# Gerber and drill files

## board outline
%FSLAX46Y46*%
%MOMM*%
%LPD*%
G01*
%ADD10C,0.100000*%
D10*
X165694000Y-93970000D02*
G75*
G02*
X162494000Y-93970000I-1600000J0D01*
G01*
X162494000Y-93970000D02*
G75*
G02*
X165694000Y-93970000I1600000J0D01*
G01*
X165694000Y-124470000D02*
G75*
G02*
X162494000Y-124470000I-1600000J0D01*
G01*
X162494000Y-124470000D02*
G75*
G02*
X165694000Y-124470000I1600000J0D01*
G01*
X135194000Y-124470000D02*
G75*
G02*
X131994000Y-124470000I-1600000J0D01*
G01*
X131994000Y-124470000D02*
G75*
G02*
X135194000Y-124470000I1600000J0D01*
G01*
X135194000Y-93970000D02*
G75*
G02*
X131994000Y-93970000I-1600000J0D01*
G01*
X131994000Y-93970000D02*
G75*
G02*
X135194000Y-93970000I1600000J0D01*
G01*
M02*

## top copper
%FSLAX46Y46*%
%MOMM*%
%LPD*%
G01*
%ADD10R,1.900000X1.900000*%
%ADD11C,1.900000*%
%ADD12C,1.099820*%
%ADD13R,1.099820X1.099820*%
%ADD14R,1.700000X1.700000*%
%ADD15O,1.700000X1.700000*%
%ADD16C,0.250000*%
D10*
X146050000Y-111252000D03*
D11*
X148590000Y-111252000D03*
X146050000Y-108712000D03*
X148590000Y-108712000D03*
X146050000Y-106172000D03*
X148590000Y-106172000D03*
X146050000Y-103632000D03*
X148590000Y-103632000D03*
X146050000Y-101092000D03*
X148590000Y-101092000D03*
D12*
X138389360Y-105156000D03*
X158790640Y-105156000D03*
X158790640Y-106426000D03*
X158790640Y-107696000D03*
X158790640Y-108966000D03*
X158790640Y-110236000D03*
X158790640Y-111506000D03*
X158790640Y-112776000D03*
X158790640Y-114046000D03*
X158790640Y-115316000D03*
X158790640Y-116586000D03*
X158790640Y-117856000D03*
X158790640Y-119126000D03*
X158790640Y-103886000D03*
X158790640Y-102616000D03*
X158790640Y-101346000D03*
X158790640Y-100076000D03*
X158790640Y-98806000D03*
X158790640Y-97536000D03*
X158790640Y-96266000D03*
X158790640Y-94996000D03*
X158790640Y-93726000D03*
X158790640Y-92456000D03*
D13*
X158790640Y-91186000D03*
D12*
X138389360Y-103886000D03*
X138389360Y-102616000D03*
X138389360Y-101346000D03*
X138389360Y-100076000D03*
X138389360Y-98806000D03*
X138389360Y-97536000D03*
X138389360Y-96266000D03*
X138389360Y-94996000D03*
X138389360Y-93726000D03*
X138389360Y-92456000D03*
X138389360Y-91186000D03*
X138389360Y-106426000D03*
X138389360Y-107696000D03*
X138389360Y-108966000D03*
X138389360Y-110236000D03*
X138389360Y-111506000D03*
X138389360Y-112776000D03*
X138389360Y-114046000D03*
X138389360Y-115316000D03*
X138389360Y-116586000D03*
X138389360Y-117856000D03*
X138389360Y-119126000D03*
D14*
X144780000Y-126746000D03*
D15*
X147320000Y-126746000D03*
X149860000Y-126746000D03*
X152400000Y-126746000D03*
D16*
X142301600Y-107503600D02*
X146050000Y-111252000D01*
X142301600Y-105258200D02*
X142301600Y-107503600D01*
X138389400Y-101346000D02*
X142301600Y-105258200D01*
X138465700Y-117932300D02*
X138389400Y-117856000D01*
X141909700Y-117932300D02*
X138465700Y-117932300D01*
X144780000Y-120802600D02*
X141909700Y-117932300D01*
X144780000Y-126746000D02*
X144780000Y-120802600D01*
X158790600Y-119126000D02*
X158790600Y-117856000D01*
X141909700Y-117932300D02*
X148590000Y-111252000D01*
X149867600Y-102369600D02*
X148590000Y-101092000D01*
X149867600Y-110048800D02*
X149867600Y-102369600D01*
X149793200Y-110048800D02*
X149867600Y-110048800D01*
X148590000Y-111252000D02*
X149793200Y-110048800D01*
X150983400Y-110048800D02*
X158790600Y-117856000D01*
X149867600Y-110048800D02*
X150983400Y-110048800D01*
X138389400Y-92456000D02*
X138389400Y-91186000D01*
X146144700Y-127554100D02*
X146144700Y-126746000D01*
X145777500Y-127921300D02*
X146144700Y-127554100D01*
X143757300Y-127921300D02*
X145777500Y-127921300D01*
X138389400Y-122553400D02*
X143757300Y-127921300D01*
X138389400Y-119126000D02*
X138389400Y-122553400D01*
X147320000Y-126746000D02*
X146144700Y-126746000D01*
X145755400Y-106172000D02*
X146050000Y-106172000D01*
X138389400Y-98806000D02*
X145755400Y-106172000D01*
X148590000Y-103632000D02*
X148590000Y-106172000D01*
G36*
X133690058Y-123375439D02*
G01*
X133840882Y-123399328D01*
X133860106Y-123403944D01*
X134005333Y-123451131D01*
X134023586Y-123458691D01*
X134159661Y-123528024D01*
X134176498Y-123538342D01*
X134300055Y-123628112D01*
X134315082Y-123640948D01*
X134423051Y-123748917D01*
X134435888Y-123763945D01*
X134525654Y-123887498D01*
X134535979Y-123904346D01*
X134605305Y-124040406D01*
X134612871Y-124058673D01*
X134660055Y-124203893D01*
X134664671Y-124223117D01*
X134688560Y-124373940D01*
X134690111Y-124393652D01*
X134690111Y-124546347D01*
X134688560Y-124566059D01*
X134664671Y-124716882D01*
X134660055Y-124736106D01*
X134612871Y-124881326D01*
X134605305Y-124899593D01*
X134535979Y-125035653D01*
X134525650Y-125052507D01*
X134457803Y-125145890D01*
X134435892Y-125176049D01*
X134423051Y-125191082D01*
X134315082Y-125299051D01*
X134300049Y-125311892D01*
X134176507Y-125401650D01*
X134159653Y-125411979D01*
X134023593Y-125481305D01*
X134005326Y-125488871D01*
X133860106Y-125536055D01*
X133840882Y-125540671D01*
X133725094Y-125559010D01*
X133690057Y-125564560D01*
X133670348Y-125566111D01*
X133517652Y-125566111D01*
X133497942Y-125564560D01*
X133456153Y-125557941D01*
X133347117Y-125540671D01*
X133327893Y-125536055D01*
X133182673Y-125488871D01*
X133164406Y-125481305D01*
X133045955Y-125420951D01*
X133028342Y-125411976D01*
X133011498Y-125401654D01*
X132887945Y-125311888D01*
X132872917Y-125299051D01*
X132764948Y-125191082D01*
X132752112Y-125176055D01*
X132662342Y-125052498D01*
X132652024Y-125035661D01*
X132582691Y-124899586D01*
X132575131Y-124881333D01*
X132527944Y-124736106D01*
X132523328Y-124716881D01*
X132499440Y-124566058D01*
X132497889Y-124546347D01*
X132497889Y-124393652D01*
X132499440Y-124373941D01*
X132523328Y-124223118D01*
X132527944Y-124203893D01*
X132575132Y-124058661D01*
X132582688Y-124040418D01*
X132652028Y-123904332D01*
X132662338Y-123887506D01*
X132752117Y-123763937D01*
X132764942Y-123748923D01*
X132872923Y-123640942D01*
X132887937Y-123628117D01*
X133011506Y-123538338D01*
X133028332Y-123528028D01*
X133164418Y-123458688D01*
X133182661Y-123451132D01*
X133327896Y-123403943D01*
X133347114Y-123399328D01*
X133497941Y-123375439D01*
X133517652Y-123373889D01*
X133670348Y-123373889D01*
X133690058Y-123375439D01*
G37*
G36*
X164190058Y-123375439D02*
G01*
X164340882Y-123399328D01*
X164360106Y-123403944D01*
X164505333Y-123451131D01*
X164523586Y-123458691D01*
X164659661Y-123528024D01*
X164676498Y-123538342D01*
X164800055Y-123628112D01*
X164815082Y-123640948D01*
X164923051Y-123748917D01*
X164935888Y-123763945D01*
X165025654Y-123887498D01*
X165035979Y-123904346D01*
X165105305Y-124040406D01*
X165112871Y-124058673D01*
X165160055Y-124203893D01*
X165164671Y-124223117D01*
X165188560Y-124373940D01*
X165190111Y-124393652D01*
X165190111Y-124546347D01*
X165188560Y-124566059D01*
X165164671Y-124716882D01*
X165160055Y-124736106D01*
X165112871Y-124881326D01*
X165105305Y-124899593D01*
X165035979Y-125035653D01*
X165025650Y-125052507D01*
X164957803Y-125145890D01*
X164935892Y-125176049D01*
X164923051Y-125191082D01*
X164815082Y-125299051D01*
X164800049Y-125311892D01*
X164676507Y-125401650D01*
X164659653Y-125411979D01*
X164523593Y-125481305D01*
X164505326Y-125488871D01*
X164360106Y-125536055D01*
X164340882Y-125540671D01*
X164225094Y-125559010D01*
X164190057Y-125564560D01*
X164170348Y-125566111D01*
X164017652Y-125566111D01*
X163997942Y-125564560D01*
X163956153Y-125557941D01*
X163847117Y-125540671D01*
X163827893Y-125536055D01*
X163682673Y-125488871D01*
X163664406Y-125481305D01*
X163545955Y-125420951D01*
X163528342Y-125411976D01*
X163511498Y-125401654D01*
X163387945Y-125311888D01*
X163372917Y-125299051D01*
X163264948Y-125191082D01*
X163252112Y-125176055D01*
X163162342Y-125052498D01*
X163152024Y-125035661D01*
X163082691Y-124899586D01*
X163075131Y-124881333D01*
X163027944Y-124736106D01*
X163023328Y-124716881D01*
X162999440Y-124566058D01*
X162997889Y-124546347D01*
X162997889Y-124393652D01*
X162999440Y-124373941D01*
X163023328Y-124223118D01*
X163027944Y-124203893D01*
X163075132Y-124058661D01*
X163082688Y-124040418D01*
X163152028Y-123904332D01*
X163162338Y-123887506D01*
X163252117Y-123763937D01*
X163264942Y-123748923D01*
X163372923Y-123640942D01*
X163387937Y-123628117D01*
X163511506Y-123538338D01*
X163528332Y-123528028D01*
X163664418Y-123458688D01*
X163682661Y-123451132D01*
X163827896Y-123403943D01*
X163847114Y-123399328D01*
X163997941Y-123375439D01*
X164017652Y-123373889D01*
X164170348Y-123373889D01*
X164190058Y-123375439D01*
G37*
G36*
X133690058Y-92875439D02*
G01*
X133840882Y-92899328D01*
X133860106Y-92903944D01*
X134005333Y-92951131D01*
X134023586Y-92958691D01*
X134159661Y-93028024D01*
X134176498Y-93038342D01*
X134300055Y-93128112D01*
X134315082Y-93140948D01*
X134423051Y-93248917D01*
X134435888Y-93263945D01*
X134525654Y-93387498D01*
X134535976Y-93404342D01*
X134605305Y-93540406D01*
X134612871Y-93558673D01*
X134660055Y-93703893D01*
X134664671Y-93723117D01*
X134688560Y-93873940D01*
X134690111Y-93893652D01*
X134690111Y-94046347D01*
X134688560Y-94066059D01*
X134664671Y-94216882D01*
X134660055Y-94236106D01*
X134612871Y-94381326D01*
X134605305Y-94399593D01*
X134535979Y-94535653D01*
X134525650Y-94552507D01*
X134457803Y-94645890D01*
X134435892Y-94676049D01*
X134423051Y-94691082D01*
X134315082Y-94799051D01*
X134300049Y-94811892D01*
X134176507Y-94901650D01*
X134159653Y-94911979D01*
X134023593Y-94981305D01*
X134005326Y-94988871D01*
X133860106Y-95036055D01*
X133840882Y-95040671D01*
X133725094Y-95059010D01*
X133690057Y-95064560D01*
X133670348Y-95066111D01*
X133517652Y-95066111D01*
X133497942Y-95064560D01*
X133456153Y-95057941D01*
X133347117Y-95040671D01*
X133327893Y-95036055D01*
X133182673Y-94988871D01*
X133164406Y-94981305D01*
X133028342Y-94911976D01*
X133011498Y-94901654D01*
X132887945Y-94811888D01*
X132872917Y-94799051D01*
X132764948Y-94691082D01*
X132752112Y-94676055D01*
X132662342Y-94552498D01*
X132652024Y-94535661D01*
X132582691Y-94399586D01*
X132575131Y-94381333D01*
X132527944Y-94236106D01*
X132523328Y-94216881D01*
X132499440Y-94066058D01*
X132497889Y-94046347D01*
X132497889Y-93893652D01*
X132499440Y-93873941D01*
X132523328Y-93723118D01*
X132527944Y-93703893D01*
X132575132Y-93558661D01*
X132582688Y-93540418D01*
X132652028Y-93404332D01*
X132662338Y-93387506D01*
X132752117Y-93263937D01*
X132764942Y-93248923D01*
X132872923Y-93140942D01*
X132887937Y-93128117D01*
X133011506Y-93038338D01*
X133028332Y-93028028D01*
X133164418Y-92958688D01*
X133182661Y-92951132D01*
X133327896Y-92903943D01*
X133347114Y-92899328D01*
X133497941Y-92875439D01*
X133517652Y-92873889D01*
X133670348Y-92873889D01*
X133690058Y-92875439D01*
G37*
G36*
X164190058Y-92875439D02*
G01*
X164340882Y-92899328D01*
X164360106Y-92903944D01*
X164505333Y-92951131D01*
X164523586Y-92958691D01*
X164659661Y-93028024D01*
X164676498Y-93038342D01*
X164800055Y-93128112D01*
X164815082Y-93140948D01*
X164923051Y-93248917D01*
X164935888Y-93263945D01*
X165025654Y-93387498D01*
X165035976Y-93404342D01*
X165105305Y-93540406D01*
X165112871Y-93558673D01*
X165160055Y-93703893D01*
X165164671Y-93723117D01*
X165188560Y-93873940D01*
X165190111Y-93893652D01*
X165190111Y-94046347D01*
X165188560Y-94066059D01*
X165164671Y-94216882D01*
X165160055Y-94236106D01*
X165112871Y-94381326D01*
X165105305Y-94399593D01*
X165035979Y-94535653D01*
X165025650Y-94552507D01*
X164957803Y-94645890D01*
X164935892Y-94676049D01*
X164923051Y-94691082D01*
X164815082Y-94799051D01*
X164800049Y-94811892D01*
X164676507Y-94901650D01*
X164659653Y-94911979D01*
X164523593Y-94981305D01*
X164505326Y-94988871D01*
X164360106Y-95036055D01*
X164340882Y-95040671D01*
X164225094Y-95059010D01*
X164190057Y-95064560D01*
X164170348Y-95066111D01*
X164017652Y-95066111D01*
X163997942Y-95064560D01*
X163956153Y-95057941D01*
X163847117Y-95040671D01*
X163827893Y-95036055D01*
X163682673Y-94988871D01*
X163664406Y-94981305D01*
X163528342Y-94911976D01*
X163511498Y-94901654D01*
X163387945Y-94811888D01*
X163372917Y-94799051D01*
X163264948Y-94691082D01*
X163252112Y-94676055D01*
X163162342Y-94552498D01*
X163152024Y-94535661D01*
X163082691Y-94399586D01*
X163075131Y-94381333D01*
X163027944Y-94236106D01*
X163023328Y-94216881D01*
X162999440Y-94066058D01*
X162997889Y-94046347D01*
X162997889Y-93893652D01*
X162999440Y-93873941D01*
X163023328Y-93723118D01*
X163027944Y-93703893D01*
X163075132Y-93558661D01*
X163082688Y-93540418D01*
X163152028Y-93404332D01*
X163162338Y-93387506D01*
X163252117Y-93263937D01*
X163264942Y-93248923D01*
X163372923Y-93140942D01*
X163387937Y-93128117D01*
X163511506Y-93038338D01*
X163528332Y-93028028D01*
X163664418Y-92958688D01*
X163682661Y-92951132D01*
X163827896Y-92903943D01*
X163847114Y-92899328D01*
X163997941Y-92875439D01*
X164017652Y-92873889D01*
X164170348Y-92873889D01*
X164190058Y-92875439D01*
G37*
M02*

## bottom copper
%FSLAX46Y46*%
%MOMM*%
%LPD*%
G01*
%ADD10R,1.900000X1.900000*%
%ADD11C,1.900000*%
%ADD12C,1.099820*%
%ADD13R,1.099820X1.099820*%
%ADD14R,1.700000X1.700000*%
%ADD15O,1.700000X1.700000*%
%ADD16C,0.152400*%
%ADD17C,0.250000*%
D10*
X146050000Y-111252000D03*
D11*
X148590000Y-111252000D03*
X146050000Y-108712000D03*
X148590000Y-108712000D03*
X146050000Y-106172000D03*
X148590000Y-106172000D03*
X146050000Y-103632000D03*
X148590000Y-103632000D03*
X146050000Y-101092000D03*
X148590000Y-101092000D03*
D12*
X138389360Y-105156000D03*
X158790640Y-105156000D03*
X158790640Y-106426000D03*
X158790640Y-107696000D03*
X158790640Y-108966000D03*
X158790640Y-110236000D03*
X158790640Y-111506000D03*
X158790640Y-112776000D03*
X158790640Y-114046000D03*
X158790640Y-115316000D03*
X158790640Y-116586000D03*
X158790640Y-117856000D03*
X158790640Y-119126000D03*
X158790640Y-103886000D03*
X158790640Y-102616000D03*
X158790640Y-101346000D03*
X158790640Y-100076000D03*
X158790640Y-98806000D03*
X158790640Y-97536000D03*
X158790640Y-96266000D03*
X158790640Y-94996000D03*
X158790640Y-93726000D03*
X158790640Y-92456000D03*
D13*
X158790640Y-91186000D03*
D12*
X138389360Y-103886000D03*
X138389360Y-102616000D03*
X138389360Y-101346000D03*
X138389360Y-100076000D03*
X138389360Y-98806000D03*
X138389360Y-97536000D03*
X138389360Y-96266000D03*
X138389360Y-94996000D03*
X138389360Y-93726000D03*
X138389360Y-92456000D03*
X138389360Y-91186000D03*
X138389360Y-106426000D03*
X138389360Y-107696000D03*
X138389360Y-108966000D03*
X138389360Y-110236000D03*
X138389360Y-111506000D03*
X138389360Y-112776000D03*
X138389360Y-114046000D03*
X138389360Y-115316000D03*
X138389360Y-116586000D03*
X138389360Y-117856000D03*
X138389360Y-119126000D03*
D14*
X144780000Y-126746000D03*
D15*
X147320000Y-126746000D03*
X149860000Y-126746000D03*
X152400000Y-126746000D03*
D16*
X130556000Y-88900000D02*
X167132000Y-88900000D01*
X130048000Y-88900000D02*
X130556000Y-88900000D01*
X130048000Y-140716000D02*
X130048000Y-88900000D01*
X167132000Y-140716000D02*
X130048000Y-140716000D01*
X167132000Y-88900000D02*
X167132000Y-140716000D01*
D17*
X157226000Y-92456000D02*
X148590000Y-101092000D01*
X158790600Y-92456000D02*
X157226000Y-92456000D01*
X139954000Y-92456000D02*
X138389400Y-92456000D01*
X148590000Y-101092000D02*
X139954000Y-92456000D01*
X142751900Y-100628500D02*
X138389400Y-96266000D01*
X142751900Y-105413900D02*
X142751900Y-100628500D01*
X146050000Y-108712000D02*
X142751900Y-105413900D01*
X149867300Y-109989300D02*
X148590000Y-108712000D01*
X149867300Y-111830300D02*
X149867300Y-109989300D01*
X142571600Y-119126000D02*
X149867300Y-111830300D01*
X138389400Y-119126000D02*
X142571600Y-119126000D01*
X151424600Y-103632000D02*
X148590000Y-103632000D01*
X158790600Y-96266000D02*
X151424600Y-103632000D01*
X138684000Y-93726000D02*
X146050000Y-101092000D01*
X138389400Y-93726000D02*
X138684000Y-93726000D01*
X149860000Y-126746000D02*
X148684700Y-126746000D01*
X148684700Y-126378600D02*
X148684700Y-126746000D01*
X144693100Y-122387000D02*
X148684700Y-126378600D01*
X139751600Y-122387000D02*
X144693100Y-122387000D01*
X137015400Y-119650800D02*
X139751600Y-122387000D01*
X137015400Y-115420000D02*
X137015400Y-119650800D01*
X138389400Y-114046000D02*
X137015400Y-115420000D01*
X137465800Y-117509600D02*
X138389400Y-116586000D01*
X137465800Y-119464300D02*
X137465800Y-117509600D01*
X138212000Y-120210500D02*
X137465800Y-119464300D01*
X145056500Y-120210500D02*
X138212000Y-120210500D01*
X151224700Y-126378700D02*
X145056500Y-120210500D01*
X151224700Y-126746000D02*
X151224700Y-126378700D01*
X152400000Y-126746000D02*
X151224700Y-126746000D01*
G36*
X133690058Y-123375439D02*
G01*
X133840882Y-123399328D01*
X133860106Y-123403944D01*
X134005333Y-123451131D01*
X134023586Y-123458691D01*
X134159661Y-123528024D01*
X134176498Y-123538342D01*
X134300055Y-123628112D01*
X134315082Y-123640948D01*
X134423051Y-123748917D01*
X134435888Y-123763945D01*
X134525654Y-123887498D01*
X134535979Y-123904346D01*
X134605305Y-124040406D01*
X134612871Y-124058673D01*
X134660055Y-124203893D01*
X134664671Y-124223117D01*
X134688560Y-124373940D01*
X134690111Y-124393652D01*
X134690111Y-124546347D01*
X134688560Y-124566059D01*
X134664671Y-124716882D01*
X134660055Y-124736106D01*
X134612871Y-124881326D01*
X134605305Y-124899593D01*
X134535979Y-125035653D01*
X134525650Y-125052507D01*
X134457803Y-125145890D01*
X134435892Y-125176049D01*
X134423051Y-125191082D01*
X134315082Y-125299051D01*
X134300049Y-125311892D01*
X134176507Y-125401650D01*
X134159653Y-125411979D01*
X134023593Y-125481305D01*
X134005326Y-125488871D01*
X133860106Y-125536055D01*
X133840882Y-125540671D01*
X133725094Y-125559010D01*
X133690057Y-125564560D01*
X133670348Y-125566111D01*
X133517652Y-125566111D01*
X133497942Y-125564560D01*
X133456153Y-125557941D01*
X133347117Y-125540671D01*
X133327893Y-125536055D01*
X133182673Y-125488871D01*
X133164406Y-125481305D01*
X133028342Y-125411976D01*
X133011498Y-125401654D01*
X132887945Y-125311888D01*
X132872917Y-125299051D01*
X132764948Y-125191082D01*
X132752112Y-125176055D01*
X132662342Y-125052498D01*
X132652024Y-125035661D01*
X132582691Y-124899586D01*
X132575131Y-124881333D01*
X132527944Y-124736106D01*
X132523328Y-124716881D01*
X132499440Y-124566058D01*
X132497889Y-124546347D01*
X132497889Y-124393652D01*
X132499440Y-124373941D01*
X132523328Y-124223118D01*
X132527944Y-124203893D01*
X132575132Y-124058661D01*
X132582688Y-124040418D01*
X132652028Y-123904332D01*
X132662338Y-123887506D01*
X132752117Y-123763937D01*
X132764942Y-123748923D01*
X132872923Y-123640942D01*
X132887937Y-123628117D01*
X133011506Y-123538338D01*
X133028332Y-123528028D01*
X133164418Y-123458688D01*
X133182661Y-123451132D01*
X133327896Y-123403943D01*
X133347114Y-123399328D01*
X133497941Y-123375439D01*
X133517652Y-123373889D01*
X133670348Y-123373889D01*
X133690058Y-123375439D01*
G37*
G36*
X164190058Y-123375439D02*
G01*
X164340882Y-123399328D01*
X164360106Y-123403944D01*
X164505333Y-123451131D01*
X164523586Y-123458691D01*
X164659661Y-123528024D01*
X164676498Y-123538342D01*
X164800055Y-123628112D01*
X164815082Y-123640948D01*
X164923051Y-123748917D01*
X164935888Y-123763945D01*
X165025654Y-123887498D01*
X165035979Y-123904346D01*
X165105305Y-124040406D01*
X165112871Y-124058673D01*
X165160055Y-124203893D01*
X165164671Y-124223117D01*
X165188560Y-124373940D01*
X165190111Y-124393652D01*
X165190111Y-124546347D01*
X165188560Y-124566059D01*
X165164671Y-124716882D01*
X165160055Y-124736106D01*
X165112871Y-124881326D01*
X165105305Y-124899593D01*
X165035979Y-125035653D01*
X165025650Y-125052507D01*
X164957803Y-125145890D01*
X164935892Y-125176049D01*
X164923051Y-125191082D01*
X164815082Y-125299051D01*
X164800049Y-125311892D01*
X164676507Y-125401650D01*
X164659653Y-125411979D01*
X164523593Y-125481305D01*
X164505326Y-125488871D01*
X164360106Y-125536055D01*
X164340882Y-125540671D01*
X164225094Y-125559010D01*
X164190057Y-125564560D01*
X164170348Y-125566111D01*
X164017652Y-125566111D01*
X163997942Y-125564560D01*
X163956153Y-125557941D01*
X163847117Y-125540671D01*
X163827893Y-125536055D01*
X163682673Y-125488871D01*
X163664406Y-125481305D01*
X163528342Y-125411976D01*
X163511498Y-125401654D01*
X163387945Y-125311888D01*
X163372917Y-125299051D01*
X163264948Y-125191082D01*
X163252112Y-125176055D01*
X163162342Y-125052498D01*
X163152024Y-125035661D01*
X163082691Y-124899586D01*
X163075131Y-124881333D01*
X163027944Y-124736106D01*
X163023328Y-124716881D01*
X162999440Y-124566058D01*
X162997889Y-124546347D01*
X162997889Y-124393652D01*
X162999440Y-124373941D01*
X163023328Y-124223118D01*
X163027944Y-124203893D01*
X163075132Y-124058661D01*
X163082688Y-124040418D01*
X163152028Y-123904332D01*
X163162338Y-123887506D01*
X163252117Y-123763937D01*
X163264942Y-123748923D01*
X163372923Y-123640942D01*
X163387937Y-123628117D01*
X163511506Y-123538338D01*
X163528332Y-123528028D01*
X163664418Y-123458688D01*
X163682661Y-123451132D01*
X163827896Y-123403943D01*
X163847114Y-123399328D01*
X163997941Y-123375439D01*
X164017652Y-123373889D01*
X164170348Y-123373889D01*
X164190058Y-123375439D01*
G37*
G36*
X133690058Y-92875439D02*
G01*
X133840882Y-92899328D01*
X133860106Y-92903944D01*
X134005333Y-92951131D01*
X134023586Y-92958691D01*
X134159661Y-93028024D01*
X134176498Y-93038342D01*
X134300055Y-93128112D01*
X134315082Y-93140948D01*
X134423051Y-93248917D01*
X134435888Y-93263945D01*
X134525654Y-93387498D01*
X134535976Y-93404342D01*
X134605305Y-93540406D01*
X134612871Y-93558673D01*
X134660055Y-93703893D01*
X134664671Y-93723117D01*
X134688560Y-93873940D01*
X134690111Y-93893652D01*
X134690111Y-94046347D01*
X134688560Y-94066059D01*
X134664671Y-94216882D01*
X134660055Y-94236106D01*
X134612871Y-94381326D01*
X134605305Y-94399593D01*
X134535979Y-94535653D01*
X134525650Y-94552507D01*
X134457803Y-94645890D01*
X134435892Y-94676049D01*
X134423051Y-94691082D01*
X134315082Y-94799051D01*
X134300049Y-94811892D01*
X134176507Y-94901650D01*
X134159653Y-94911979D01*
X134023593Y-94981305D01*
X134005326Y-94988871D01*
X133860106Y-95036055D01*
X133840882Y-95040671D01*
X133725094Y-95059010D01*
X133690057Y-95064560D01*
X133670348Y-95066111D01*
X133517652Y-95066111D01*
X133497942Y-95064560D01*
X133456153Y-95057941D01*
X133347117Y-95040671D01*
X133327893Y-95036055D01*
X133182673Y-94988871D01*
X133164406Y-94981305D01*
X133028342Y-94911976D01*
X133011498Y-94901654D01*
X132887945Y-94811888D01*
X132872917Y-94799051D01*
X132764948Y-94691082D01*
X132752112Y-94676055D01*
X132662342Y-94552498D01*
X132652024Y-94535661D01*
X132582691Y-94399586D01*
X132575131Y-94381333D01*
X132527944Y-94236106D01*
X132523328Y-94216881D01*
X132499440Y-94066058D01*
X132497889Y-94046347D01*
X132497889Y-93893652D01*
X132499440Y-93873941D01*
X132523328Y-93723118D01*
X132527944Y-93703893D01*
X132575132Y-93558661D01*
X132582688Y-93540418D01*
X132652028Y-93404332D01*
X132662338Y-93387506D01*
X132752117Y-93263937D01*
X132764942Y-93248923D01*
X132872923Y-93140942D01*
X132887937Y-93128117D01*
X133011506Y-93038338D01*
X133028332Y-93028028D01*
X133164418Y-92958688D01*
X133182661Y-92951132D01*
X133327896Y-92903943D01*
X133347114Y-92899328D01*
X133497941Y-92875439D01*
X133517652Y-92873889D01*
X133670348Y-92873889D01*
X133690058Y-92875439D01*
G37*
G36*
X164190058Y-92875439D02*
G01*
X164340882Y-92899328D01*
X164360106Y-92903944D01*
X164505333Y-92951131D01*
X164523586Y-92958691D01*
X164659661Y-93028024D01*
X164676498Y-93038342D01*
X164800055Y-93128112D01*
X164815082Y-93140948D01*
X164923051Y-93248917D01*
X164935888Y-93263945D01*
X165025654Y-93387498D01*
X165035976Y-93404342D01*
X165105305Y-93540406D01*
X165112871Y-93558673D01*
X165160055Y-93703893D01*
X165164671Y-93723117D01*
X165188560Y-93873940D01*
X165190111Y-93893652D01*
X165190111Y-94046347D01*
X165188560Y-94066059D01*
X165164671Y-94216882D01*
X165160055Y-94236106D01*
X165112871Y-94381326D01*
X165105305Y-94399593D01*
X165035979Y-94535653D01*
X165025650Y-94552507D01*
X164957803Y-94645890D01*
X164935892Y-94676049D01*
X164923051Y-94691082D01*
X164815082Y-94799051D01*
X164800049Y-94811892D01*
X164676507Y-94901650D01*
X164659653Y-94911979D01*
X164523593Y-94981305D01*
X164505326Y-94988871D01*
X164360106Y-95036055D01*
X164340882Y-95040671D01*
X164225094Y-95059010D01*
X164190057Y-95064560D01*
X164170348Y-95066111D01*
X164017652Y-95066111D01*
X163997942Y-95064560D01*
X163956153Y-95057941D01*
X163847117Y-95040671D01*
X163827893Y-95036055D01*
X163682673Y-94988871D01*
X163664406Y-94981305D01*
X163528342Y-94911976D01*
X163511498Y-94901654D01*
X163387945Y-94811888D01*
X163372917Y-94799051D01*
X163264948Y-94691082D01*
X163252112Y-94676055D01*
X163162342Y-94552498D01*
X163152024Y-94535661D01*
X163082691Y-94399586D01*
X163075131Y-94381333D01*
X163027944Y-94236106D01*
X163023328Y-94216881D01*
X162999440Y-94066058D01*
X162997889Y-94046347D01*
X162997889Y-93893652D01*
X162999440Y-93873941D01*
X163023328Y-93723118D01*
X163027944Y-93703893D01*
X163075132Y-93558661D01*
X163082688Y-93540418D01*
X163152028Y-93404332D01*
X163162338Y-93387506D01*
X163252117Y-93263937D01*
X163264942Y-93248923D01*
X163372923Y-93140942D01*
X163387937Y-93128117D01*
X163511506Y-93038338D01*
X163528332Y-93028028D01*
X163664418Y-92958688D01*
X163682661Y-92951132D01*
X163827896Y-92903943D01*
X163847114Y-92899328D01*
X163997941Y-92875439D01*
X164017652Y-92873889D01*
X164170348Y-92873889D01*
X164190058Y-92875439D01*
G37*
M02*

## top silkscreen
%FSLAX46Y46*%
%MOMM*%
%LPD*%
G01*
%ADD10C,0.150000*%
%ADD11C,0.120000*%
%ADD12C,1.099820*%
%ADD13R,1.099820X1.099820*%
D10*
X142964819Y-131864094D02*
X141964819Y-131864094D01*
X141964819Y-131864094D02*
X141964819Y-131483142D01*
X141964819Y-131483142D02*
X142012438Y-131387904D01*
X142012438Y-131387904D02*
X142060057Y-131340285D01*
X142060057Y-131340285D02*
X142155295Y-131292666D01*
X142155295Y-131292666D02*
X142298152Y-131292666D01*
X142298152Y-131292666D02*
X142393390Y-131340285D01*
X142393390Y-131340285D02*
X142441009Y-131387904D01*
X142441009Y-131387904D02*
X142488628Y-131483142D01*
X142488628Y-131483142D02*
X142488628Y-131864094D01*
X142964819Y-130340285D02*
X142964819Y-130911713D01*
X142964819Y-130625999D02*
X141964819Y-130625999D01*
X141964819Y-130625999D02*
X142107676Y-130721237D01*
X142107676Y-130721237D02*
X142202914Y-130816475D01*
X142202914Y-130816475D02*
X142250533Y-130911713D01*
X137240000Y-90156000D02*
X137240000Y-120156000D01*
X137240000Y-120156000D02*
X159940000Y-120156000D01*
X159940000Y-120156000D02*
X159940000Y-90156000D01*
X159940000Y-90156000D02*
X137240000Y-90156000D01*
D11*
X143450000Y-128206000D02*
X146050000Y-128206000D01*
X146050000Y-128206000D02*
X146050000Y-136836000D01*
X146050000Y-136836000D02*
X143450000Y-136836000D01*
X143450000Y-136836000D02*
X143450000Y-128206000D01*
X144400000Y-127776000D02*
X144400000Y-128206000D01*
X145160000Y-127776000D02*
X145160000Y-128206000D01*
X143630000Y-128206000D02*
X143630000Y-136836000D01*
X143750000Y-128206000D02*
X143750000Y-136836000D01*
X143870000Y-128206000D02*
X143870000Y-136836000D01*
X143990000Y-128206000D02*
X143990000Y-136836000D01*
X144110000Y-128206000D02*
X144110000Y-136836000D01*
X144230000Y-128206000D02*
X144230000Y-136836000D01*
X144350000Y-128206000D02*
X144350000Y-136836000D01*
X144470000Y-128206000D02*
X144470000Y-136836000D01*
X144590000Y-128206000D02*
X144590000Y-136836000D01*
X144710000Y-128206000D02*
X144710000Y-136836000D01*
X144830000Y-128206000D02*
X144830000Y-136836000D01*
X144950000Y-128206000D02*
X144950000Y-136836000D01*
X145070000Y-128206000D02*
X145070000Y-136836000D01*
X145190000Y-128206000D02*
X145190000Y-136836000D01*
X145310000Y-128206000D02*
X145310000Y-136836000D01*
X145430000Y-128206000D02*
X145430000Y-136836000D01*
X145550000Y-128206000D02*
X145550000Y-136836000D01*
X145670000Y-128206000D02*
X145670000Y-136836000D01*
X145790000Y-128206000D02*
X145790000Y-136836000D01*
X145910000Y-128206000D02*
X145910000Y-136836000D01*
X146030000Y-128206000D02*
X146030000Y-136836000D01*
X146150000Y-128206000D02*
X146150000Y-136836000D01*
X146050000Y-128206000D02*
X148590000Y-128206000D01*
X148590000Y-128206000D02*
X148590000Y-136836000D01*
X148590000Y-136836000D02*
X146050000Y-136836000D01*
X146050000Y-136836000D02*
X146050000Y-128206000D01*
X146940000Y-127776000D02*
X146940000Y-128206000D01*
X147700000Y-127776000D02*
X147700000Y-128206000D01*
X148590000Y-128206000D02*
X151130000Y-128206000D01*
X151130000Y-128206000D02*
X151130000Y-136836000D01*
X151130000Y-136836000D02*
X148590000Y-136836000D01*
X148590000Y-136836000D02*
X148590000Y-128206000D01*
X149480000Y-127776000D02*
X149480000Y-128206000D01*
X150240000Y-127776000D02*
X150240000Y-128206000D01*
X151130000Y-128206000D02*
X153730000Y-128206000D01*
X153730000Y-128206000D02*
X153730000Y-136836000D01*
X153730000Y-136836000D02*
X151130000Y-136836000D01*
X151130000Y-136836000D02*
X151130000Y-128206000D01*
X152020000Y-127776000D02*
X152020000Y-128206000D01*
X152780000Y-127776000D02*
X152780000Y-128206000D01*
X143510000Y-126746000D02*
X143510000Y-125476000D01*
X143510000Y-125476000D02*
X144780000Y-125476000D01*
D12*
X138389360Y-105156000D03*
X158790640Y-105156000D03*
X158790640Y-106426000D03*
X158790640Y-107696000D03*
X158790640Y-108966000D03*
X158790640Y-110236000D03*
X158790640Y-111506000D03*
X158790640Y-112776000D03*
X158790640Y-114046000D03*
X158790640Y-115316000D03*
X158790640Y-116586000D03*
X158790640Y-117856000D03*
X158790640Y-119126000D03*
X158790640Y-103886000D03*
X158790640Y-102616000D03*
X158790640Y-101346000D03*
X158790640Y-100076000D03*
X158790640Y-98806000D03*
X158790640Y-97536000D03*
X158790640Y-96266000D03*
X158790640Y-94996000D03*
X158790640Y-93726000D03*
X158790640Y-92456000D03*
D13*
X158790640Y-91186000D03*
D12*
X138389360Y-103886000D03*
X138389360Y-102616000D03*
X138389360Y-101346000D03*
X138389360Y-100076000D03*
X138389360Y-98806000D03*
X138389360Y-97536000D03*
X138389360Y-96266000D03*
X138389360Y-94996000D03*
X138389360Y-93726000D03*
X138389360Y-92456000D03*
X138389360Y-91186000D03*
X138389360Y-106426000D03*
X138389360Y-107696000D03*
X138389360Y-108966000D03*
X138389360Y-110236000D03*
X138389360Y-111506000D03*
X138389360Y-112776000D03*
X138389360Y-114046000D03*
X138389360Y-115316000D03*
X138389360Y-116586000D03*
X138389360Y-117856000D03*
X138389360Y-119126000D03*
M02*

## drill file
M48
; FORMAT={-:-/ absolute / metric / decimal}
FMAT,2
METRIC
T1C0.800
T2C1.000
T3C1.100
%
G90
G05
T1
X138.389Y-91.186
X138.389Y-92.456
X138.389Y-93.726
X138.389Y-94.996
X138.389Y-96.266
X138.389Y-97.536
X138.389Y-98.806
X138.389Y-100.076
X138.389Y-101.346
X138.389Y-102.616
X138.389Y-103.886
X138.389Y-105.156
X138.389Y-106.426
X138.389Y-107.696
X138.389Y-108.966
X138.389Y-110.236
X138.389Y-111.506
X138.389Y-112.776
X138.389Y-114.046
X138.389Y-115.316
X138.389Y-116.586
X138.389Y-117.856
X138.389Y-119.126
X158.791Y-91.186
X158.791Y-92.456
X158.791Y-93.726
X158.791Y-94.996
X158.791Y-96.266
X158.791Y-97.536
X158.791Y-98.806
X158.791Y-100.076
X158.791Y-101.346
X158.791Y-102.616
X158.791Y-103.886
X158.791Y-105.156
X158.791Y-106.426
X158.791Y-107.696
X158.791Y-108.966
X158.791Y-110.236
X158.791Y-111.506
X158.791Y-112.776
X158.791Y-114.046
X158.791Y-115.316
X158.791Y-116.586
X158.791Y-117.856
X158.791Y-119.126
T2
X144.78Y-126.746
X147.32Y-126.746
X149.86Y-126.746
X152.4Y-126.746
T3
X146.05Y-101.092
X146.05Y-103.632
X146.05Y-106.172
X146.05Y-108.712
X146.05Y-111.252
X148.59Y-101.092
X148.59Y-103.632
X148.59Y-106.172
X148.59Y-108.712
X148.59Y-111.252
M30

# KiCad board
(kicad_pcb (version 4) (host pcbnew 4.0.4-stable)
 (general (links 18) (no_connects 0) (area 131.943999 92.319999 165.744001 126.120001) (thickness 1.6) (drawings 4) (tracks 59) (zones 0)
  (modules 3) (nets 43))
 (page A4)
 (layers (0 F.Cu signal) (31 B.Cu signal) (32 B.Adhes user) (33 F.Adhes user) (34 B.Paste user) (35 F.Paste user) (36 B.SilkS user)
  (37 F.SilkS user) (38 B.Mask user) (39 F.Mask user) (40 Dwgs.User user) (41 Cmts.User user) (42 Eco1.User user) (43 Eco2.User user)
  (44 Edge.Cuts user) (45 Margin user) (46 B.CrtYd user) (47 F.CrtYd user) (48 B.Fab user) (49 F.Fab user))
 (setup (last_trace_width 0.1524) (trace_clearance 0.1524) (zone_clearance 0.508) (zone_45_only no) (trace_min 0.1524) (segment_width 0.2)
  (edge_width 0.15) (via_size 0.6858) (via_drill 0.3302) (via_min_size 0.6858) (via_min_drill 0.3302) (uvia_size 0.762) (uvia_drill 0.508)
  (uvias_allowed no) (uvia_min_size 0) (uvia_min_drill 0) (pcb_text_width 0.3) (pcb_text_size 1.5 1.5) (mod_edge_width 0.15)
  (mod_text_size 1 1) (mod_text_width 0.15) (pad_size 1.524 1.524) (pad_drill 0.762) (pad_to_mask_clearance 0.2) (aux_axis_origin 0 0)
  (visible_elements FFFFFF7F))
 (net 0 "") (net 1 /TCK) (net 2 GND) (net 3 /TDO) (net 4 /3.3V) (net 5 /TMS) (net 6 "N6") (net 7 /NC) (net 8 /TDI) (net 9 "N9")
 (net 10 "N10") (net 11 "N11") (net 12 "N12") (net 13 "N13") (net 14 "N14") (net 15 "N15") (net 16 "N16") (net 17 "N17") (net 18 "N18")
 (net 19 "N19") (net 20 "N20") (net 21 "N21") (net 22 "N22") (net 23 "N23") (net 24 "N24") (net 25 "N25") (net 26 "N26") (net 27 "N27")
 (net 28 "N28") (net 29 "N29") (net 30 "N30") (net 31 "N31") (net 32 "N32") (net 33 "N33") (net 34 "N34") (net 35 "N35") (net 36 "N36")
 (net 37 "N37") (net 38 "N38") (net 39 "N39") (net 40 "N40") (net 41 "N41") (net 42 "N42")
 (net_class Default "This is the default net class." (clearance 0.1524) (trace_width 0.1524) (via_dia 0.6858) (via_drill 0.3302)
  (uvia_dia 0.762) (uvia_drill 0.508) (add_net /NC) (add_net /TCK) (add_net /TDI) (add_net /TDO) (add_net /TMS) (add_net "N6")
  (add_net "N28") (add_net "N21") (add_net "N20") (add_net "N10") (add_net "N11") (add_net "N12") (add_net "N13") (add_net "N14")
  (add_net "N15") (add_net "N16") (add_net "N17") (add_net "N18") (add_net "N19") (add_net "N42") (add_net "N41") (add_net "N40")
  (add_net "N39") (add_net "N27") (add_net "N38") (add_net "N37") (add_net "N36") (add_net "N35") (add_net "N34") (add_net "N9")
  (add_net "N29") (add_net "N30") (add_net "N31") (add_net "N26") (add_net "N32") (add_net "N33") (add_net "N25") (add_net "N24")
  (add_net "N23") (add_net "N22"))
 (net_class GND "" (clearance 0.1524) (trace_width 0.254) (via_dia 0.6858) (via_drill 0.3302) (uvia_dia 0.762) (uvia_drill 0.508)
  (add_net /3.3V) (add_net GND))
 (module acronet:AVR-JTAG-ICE (layer B.Cu) (at 147.32 106.172 90)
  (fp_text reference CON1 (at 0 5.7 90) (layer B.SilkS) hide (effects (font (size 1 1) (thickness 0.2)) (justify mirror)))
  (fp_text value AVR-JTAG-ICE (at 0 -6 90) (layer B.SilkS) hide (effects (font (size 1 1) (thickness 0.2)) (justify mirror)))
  (pad 1 thru_hole rect (at -5.08 -1.27 90) (size 1.9 1.9) (drill 1.1) (layers *.Cu *.Mask B.SilkS) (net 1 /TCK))
  (pad 2 thru_hole circle (at -5.08 1.27 90) (size 1.9 1.9) (drill 1.1) (layers *.Cu *.Mask B.SilkS) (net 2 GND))
  (pad 3 thru_hole circle (at -2.54 -1.27 90) (size 1.9 1.9) (drill 1.1) (layers *.Cu *.Mask B.SilkS) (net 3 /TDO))
  (pad 4 thru_hole circle (at -2.54 1.27 90) (size 1.9 1.9) (drill 1.1) (layers *.Cu *.Mask B.SilkS) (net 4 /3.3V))
  (pad 5 thru_hole circle (at 0 -1.27 90) (size 1.9 1.9) (drill 1.1) (layers *.Cu *.Mask B.SilkS) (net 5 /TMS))
  (pad 6 thru_hole circle (at 0 1.27 90) (size 1.9 1.9) (drill 1.1) (layers *.Cu *.Mask B.SilkS) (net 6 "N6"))
  (pad 7 thru_hole circle (at 2.54 -1.27 90) (size 1.9 1.9) (drill 1.1) (layers *.Cu *.Mask B.SilkS) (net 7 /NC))
  (pad 8 thru_hole circle (at 2.54 1.27 90) (size 1.9 1.9) (drill 1.1) (layers *.Cu *.Mask B.SilkS) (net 6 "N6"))
  (pad 9 thru_hole circle (at 5.08 -1.27 90) (size 1.9 1.9) (drill 1.1) (layers *.Cu *.Mask B.SilkS) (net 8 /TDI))
  (pad 10 thru_hole circle (at 5.08 1.27 90) (size 1.9 1.9) (drill 1.1) (layers *.Cu *.Mask B.SilkS) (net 2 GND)))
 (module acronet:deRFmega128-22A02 (layer F.Cu) (at 148.59 105.156 90)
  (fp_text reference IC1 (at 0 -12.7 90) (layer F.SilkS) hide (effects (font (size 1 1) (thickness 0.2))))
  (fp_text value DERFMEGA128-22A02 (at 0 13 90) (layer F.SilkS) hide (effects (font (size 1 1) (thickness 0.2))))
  (fp_line (start 15 -11.35) (end -15 -11.35) (layer F.SilkS) (width 0.15))
  (fp_line (start -15 -11.35) (end -15 11.35) (layer F.SilkS) (width 0.15))
  (fp_line (start -15 11.35) (end 15 11.35) (layer F.SilkS) (width 0.15))
  (fp_line (start 15 11.35) (end 15 -11.35) (layer F.SilkS) (width 0.15))
  (pad 35 thru_hole circle (at 0 -10.20064 90) (size 1.09982 1.09982) (drill 0.8001) (layers *.Cu *.Mask F.SilkS) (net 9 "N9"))
  (pad 12 thru_hole circle (at 0 10.20064 90) (size 1.09982 1.09982) (drill 0.8001) (layers *.Cu *.Mask F.SilkS) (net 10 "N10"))
  (pad 13 thru_hole circle (at -1.27 10.20064 90) (size 1.09982 1.09982) (drill 0.8001) (layers *.Cu *.Mask F.SilkS) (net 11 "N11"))
  (pad 14 thru_hole circle (at -2.54 10.20064 90) (size 1.09982 1.09982) (drill 0.8001) (layers *.Cu *.Mask F.SilkS) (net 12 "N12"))
  (pad 15 thru_hole circle (at -3.81 10.20064 90) (size 1.09982 1.09982) (drill 0.8001) (layers *.Cu *.Mask F.SilkS) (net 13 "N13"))
  (pad 16 thru_hole circle (at -5.08 10.20064 90) (size 1.09982 1.09982) (drill 0.8001) (layers *.Cu *.Mask F.SilkS) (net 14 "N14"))
  (pad 17 thru_hole circle (at -6.35 10.20064 90) (size 1.09982 1.09982) (drill 0.8001) (layers *.Cu *.Mask F.SilkS) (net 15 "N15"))
  (pad 18 thru_hole circle (at -7.62 10.20064 90) (size 1.09982 1.09982) (drill 0.8001) (layers *.Cu *.Mask F.SilkS) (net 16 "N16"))
  (pad 19 thru_hole circle (at -8.89 10.20064 90) (size 1.09982 1.09982) (drill 0.8001) (layers *.Cu *.Mask F.SilkS) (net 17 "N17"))
  (pad 20 thru_hole circle (at -10.16 10.20064 90) (size 1.09982 1.09982) (drill 0.8001) (layers *.Cu *.Mask F.SilkS) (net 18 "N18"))
  (pad 21 thru_hole circle (at -11.43 10.20064 90) (size 1.09982 1.09982) (drill 0.8001) (layers *.Cu *.Mask F.SilkS) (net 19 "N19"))
  (pad 22 thru_hole circle (at -12.7 10.20064 90) (size 1.09982 1.09982) (drill 0.8001) (layers *.Cu *.Mask F.SilkS) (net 2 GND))
  (pad 23 thru_hole circle (at -13.97 10.20064 90) (size 1.09982 1.09982) (drill 0.8001) (layers *.Cu *.Mask F.SilkS) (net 2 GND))
  (pad 11 thru_hole circle (at 1.27 10.20064 90) (size 1.09982 1.09982) (drill 0.8001) (layers *.Cu *.Mask F.SilkS) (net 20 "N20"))
  (pad 10 thru_hole circle (at 2.54 10.20064 90) (size 1.09982 1.09982) (drill 0.8001) (layers *.Cu *.Mask F.SilkS) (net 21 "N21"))
  (pad 9 thru_hole circle (at 3.81 10.20064 90) (size 1.09982 1.09982) (drill 0.8001) (layers *.Cu *.Mask F.SilkS) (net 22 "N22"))
  (pad 8 thru_hole circle (at 5.08 10.20064 90) (size 1.09982 1.09982) (drill 0.8001) (layers *.Cu *.Mask F.SilkS) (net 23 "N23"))
  (pad 7 thru_hole circle (at 6.35 10.20064 90) (size 1.09982 1.09982) (drill 0.8001) (layers *.Cu *.Mask F.SilkS) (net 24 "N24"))
  (pad 6 thru_hole circle (at 7.62 10.20064 90) (size 1.09982 1.09982) (drill 0.8001) (layers *.Cu *.Mask F.SilkS) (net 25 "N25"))
  (pad 5 thru_hole circle (at 8.89 10.20064 90) (size 1.09982 1.09982) (drill 0.8001) (layers *.Cu *.Mask F.SilkS) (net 6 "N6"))
  (pad 4 thru_hole circle (at 10.16 10.20064 90) (size 1.09982 1.09982) (drill 0.8001) (layers *.Cu *.Mask F.SilkS) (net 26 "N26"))
  (pad 3 thru_hole circle (at 11.43 10.20064 90) (size 1.09982 1.09982) (drill 0.8001) (layers *.Cu *.Mask F.SilkS) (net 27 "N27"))
  (pad 2 thru_hole circle (at 12.7 10.20064 90) (size 1.09982 1.09982) (drill 0.8001) (layers *.Cu *.Mask F.SilkS) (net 2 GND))
  (pad 1 thru_hole rect (at 13.97 10.20064 90) (size 1.09982 1.09982) (drill 0.8001) (layers *.Cu *.Mask F.SilkS) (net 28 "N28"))
  (pad 36 thru_hole circle (at 1.27 -10.20064 90) (size 1.09982 1.09982) (drill 0.8001) (layers *.Cu *.Mask F.SilkS) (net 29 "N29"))
  (pad 37 thru_hole circle (at 2.54 -10.20064 90) (size 1.09982 1.09982) (drill 0.8001) (layers *.Cu *.Mask F.SilkS) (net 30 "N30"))
  (pad 38 thru_hole circle (at 3.81 -10.20064 90) (size 1.09982 1.09982) (drill 0.8001) (layers *.Cu *.Mask F.SilkS) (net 1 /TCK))
  (pad 39 thru_hole circle (at 5.08 -10.20064 90) (size 1.09982 1.09982) (drill 0.8001) (layers *.Cu *.Mask F.SilkS) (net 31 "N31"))
  (pad 40 thru_hole circle (at 6.35 -10.20064 90) (size 1.09982 1.09982) (drill 0.8001) (layers *.Cu *.Mask F.SilkS) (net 5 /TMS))
  (pad 41 thru_hole circle (at 7.62 -10.20064 90) (size 1.09982 1.09982) (drill 0.8001) (layers *.Cu *.Mask F.SilkS) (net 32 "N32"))
  (pad 42 thru_hole circle (at 8.89 -10.20064 90) (size 1.09982 1.09982) (drill 0.8001) (layers *.Cu *.Mask F.SilkS) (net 3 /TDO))
  (pad 43 thru_hole circle (at 10.16 -10.20064 90) (size 1.09982 1.09982) (drill 0.8001) (layers *.Cu *.Mask F.SilkS) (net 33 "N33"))
  (pad 44 thru_hole circle (at 11.43 -10.20064 90) (size 1.09982 1.09982) (drill 0.8001) (layers *.Cu *.Mask F.SilkS) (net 8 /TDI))
  (pad 45 thru_hole circle (at 12.7 -10.20064 90) (size 1.09982 1.09982) (drill 0.8001) (layers *.Cu *.Mask F.SilkS) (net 2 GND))
  (pad 46 thru_hole circle (at 13.97 -10.20064 90) (size 1.09982 1.09982) (drill 0.8001) (layers *.Cu *.Mask F.SilkS) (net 2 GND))
  (pad 34 thru_hole circle (at -1.27 -10.20064 90) (size 1.09982 1.09982) (drill 0.8001) (layers *.Cu *.Mask F.SilkS) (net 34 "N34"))
  (pad 33 thru_hole circle (at -2.54 -10.20064 90) (size 1.09982 1.09982) (drill 0.8001) (layers *.Cu *.Mask F.SilkS) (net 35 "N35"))
  (pad 32 thru_hole circle (at -3.81 -10.20064 90) (size 1.09982 1.09982) (drill 0.8001) (layers *.Cu *.Mask F.SilkS) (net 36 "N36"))
  (pad 31 thru_hole circle (at -5.08 -10.20064 90) (size 1.09982 1.09982) (drill 0.8001) (layers *.Cu *.Mask F.SilkS) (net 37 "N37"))
  (pad 30 thru_hole circle (at -6.35 -10.20064 90) (size 1.09982 1.09982) (drill 0.8001) (layers *.Cu *.Mask F.SilkS) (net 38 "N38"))
  (pad 29 thru_hole circle (at -7.62 -10.20064 90) (size 1.09982 1.09982) (drill 0.8001) (layers *.Cu *.Mask F.SilkS) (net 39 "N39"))
  (pad 28 thru_hole circle (at -8.89 -10.20064 90) (size 1.09982 1.09982) (drill 0.8001) (layers *.Cu *.Mask F.SilkS) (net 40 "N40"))
  (pad 27 thru_hole circle (at -10.16 -10.20064 90) (size 1.09982 1.09982) (drill 0.8001) (layers *.Cu *.Mask F.SilkS) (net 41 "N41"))
  (pad 26 thru_hole circle (at -11.43 -10.20064 90) (size 1.09982 1.09982) (drill 0.8001) (layers *.Cu *.Mask F.SilkS) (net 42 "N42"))
  (pad 25 thru_hole circle (at -12.7 -10.20064 90) (size 1.09982 1.09982) (drill 0.8001) (layers *.Cu *.Mask F.SilkS) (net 2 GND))
  (pad 24 thru_hole circle (at -13.97 -10.20064 90) (size 1.09982 1.09982) (drill 0.8001) (layers *.Cu *.Mask F.SilkS) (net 4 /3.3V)))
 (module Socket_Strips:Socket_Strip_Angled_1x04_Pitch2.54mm (layer F.Cu) (at 144.78 126.746 90)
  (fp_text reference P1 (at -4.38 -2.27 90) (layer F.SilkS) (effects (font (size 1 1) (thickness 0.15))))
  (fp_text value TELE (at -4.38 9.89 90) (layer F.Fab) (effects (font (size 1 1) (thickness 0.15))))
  (fp_line (start -1.46 -1.33) (end -1.46 1.27) (layer F.SilkS) (width 0.12))
  (fp_line (start -1.46 1.27) (end -10.09 1.27) (layer F.SilkS) (width 0.12))
  (fp_line (start -10.09 1.27) (end -10.09 -1.33) (layer F.SilkS) (width 0.12))
  (fp_line (start -10.09 -1.33) (end -1.46 -1.33) (layer F.SilkS) (width 0.12))
  (fp_line (start -1.03 -0.38) (end -1.46 -0.38) (layer F.SilkS) (width 0.12))
  (fp_line (start -1.03 0.38) (end -1.46 0.38) (layer F.SilkS) (width 0.12))
  (fp_line (start -1.46 -1.15) (end -10.09 -1.15) (layer F.SilkS) (width 0.12))
  (fp_line (start -1.46 -1.03) (end -10.09 -1.03) (layer F.SilkS) (width 0.12))
  (fp_line (start -1.46 -0.91) (end -10.09 -0.91) (layer F.SilkS) (width 0.12))
  (fp_line (start -1.46 -0.79) (end -10.09 -0.79) (layer F.SilkS) (width 0.12))
  (fp_line (start -1.46 -0.67) (end -10.09 -0.67) (layer F.SilkS) (width 0.12))
  (fp_line (start -1.46 -0.55) (end -10.09 -0.55) (layer F.SilkS) (width 0.12))
  (fp_line (start -1.46 -0.43) (end -10.09 -0.43) (layer F.SilkS) (width 0.12))
  (fp_line (start -1.46 -0.31) (end -10.09 -0.31) (layer F.SilkS) (width 0.12))
  (fp_line (start -1.46 -0.19) (end -10.09 -0.19) (layer F.SilkS) (width 0.12))
  (fp_line (start -1.46 -0.07) (end -10.09 -0.07) (layer F.SilkS) (width 0.12))
  (fp_line (start -1.46 0.05) (end -10.09 0.05) (layer F.SilkS) (width 0.12))
  (fp_line (start -1.46 0.17) (end -10.09 0.17) (layer F.SilkS) (width 0.12))
  (fp_line (start -1.46 0.29) (end -10.09 0.29) (layer F.SilkS) (width 0.12))
  (fp_line (start -1.46 0.41) (end -10.09 0.41) (layer F.SilkS) (width 0.12))
  (fp_line (start -1.46 0.53) (end -10.09 0.53) (layer F.SilkS) (width 0.12))
  (fp_line (start -1.46 0.65) (end -10.09 0.65) (layer F.SilkS) (width 0.12))
  (fp_line (start -1.46 0.77) (end -10.09 0.77) (layer F.SilkS) (width 0.12))
  (fp_line (start -1.46 0.89) (end -10.09 0.89) (layer F.SilkS) (width 0.12))
  (fp_line (start -1.46 1.01) (end -10.09 1.01) (layer F.SilkS) (width 0.12))
  (fp_line (start -1.46 1.13) (end -10.09 1.13) (layer F.SilkS) (width 0.12))
  (fp_line (start -1.46 1.25) (end -10.09 1.25) (layer F.SilkS) (width 0.12))
  (fp_line (start -1.46 1.37) (end -10.09 1.37) (layer F.SilkS) (width 0.12))
  (fp_line (start -1.46 1.27) (end -1.46 3.81) (layer F.SilkS) (width 0.12))
  (fp_line (start -1.46 3.81) (end -10.09 3.81) (layer F.SilkS) (width 0.12))
  (fp_line (start -10.09 3.81) (end -10.09 1.27) (layer F.SilkS) (width 0.12))
  (fp_line (start -10.09 1.27) (end -1.46 1.27) (layer F.SilkS) (width 0.12))
  (fp_line (start -1.03 2.16) (end -1.46 2.16) (layer F.SilkS) (width 0.12))
  (fp_line (start -1.03 2.92) (end -1.46 2.92) (layer F.SilkS) (width 0.12))
  (fp_line (start -1.46 3.81) (end -1.46 6.35) (layer F.SilkS) (width 0.12))
  (fp_line (start -1.46 6.35) (end -10.09 6.35) (layer F.SilkS) (width 0.12))
  (fp_line (start -10.09 6.35) (end -10.09 3.81) (layer F.SilkS) (width 0.12))
  (fp_line (start -10.09 3.81) (end -1.46 3.81) (layer F.SilkS) (width 0.12))
  (fp_line (start -1.03 4.7) (end -1.46 4.7) (layer F.SilkS) (width 0.12))
  (fp_line (start -1.03 5.46) (end -1.46 5.46) (layer F.SilkS) (width 0.12))
  (fp_line (start -1.46 6.35) (end -1.46 8.95) (layer F.SilkS) (width 0.12))
  (fp_line (start -1.46 8.95) (end -10.09 8.95) (layer F.SilkS) (width 0.12))
  (fp_line (start -10.09 8.95) (end -10.09 6.35) (layer F.SilkS) (width 0.12))
  (fp_line (start -10.09 6.35) (end -1.46 6.35) (layer F.SilkS) (width 0.12))
  (fp_line (start -1.03 7.24) (end -1.46 7.24) (layer F.SilkS) (width 0.12))
  (fp_line (start -1.03 8) (end -1.46 8) (layer F.SilkS) (width 0.12))
  (fp_line (start 0 -1.27) (end 1.27 -1.27) (layer F.SilkS) (width 0.12))
  (fp_line (start 1.27 -1.27) (end 1.27 0) (layer F.SilkS) (width 0.12))
  (pad 1 thru_hole rect (at 0 0 90) (size 1.7 1.7) (drill 1) (layers *.Cu *.Mask) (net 2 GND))
  (pad 2 thru_hole oval (at 0 2.54 90) (size 1.7 1.7) (drill 1) (layers *.Cu *.Mask) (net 4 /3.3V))
  (pad 3 thru_hole oval (at 0 5.08 90) (size 1.7 1.7) (drill 1) (layers *.Cu *.Mask) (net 40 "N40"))
  (pad 4 thru_hole oval (at 0 7.62 90) (size 1.7 1.7) (drill 1) (layers *.Cu *.Mask) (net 42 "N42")))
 (gr_circle (center 164.094 93.97) (end 165.694 93.97) (layer Edge.Cuts) (width 0.1))
 (gr_circle (center 164.094 124.47) (end 165.694 124.47) (layer Edge.Cuts) (width 0.1))
 (gr_circle (center 133.594 124.47) (end 135.194 124.47) (layer Edge.Cuts) (width 0.1))
 (gr_circle (center 133.594 93.97) (end 135.194 93.97) (layer Edge.Cuts) (width 0.1))
 (segment (start 130.556 88.9) (end 167.132 88.9) (width 0.1524) (layer B.Cu) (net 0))
 (segment (start 130.048 88.9) (end 130.556 88.9) (width 0.1524) (layer B.Cu) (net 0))
 (segment (start 130.048 140.716) (end 130.048 88.9) (width 0.1524) (layer B.Cu) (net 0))
 (segment (start 167.132 140.716) (end 130.048 140.716) (width 0.1524) (layer B.Cu) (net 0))
 (segment (start 167.132 88.9) (end 167.132 140.716) (width 0.1524) (layer B.Cu) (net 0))
 (segment (start 142.3016 107.5036) (end 146.05 111.252) (width 0.25) (layer F.Cu) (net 1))
 (segment (start 142.3016 105.2582) (end 142.3016 107.5036) (width 0.25) (layer F.Cu) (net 1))
 (segment (start 138.3894 101.346) (end 142.3016 105.2582) (width 0.25) (layer F.Cu) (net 1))
 (segment (start 157.226 92.456) (end 148.59 101.092) (width 0.25) (layer B.Cu) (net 2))
 (segment (start 158.7906 92.456) (end 157.226 92.456) (width 0.25) (layer B.Cu) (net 2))
 (segment (start 139.954 92.456) (end 138.3894 92.456) (width 0.25) (layer B.Cu) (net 2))
 (segment (start 148.59 101.092) (end 139.954 92.456) (width 0.25) (layer B.Cu) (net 2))
 (segment (start 138.4657 117.9323) (end 138.3894 117.856) (width 0.25) (layer F.Cu) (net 2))
 (segment (start 141.9097 117.9323) (end 138.4657 117.9323) (width 0.25) (layer F.Cu) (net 2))
 (segment (start 144.78 120.8026) (end 141.9097 117.9323) (width 0.25) (layer F.Cu) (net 2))
 (segment (start 144.78 126.746) (end 144.78 120.8026) (width 0.25) (layer F.Cu) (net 2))
 (segment (start 158.7906 119.126) (end 158.7906 117.856) (width 0.25) (layer F.Cu) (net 2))
 (segment (start 141.9097 117.9323) (end 148.59 111.252) (width 0.25) (layer F.Cu) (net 2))
 (segment (start 149.8676 102.3696) (end 148.59 101.092) (width 0.25) (layer F.Cu) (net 2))
 (segment (start 149.8676 110.0488) (end 149.8676 102.3696) (width 0.25) (layer F.Cu) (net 2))
 (segment (start 149.7932 110.0488) (end 149.8676 110.0488) (width 0.25) (layer F.Cu) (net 2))
 (segment (start 148.59 111.252) (end 149.7932 110.0488) (width 0.25) (layer F.Cu) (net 2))
 (segment (start 150.9834 110.0488) (end 158.7906 117.856) (width 0.25) (layer F.Cu) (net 2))
 (segment (start 149.8676 110.0488) (end 150.9834 110.0488) (width 0.25) (layer F.Cu) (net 2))
 (segment (start 138.3894 92.456) (end 138.3894 91.186) (width 0.25) (layer F.Cu) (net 2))
 (segment (start 142.7519 100.6285) (end 138.3894 96.266) (width 0.25) (layer B.Cu) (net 3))
 (segment (start 142.7519 105.4139) (end 142.7519 100.6285) (width 0.25) (layer B.Cu) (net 3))
 (segment (start 146.05 108.712) (end 142.7519 105.4139) (width 0.25) (layer B.Cu) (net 3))
 (segment (start 146.1447 127.5541) (end 146.1447 126.746) (width 0.25) (layer F.Cu) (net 4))
 (segment (start 145.7775 127.9213) (end 146.1447 127.5541) (width 0.25) (layer F.Cu) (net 4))
 (segment (start 143.7573 127.9213) (end 145.7775 127.9213) (width 0.25) (layer F.Cu) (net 4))
 (segment (start 138.3894 122.5534) (end 143.7573 127.9213) (width 0.25) (layer F.Cu) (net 4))
 (segment (start 138.3894 119.126) (end 138.3894 122.5534) (width 0.25) (layer F.Cu) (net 4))
 (segment (start 147.32 126.746) (end 146.1447 126.746) (width 0.25) (layer F.Cu) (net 4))
 (segment (start 149.8673 109.9893) (end 148.59 108.712) (width 0.25) (layer B.Cu) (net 4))
 (segment (start 149.8673 111.8303) (end 149.8673 109.9893) (width 0.25) (layer B.Cu) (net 4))
 (segment (start 142.5716 119.126) (end 149.8673 111.8303) (width 0.25) (layer B.Cu) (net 4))
 (segment (start 138.3894 119.126) (end 142.5716 119.126) (width 0.25) (layer B.Cu) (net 4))
 (segment (start 145.7554 106.172) (end 146.05 106.172) (width 0.25) (layer F.Cu) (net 5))
 (segment (start 138.3894 98.806) (end 145.7554 106.172) (width 0.25) (layer F.Cu) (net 5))
 (segment (start 151.4246 103.632) (end 148.59 103.632) (width 0.25) (layer B.Cu) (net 6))
 (segment (start 158.7906 96.266) (end 151.4246 103.632) (width 0.25) (layer B.Cu) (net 6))
 (segment (start 148.59 103.632) (end 148.59 106.172) (width 0.25) (layer F.Cu) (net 6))
 (segment (start 138.684 93.726) (end 146.05 101.092) (width 0.25) (layer B.Cu) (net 8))
 (segment (start 138.3894 93.726) (end 138.684 93.726) (width 0.25) (layer B.Cu) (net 8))
 (segment (start 149.86 126.746) (end 148.6847 126.746) (width 0.25) (layer B.Cu) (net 40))
 (segment (start 148.6847 126.3786) (end 148.6847 126.746) (width 0.25) (layer B.Cu) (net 40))
 (segment (start 144.6931 122.387) (end 148.6847 126.3786) (width 0.25) (layer B.Cu) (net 40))
 (segment (start 139.7516 122.387) (end 144.6931 122.387) (width 0.25) (layer B.Cu) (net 40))
 (segment (start 137.0154 119.6508) (end 139.7516 122.387) (width 0.25) (layer B.Cu) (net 40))
 (segment (start 137.0154 115.42) (end 137.0154 119.6508) (width 0.25) (layer B.Cu) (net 40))
 (segment (start 138.3894 114.046) (end 137.0154 115.42) (width 0.25) (layer B.Cu) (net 40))
 (segment (start 137.4658 117.5096) (end 138.3894 116.586) (width 0.25) (layer B.Cu) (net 42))
 (segment (start 137.4658 119.4643) (end 137.4658 117.5096) (width 0.25) (layer B.Cu) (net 42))
 (segment (start 138.212 120.2105) (end 137.4658 119.4643) (width 0.25) (layer B.Cu) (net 42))
 (segment (start 145.0565 120.2105) (end 138.212 120.2105) (width 0.25) (layer B.Cu) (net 42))
 (segment (start 151.2247 126.3787) (end 145.0565 120.2105) (width 0.25) (layer B.Cu) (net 42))
 (segment (start 151.2247 126.746) (end 151.2247 126.3787) (width 0.25) (layer B.Cu) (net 42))
 (segment (start 152.4 126.746) (end 151.2247 126.746) (width 0.25) (layer B.Cu) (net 42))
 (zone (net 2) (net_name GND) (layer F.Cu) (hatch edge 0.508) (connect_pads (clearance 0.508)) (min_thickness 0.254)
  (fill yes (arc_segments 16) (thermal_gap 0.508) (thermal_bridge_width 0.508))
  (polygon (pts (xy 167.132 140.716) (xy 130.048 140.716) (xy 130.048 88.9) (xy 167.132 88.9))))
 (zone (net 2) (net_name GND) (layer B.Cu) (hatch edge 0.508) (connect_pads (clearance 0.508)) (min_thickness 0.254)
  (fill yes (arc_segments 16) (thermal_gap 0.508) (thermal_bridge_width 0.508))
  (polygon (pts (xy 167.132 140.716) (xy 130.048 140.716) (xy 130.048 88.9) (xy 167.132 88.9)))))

